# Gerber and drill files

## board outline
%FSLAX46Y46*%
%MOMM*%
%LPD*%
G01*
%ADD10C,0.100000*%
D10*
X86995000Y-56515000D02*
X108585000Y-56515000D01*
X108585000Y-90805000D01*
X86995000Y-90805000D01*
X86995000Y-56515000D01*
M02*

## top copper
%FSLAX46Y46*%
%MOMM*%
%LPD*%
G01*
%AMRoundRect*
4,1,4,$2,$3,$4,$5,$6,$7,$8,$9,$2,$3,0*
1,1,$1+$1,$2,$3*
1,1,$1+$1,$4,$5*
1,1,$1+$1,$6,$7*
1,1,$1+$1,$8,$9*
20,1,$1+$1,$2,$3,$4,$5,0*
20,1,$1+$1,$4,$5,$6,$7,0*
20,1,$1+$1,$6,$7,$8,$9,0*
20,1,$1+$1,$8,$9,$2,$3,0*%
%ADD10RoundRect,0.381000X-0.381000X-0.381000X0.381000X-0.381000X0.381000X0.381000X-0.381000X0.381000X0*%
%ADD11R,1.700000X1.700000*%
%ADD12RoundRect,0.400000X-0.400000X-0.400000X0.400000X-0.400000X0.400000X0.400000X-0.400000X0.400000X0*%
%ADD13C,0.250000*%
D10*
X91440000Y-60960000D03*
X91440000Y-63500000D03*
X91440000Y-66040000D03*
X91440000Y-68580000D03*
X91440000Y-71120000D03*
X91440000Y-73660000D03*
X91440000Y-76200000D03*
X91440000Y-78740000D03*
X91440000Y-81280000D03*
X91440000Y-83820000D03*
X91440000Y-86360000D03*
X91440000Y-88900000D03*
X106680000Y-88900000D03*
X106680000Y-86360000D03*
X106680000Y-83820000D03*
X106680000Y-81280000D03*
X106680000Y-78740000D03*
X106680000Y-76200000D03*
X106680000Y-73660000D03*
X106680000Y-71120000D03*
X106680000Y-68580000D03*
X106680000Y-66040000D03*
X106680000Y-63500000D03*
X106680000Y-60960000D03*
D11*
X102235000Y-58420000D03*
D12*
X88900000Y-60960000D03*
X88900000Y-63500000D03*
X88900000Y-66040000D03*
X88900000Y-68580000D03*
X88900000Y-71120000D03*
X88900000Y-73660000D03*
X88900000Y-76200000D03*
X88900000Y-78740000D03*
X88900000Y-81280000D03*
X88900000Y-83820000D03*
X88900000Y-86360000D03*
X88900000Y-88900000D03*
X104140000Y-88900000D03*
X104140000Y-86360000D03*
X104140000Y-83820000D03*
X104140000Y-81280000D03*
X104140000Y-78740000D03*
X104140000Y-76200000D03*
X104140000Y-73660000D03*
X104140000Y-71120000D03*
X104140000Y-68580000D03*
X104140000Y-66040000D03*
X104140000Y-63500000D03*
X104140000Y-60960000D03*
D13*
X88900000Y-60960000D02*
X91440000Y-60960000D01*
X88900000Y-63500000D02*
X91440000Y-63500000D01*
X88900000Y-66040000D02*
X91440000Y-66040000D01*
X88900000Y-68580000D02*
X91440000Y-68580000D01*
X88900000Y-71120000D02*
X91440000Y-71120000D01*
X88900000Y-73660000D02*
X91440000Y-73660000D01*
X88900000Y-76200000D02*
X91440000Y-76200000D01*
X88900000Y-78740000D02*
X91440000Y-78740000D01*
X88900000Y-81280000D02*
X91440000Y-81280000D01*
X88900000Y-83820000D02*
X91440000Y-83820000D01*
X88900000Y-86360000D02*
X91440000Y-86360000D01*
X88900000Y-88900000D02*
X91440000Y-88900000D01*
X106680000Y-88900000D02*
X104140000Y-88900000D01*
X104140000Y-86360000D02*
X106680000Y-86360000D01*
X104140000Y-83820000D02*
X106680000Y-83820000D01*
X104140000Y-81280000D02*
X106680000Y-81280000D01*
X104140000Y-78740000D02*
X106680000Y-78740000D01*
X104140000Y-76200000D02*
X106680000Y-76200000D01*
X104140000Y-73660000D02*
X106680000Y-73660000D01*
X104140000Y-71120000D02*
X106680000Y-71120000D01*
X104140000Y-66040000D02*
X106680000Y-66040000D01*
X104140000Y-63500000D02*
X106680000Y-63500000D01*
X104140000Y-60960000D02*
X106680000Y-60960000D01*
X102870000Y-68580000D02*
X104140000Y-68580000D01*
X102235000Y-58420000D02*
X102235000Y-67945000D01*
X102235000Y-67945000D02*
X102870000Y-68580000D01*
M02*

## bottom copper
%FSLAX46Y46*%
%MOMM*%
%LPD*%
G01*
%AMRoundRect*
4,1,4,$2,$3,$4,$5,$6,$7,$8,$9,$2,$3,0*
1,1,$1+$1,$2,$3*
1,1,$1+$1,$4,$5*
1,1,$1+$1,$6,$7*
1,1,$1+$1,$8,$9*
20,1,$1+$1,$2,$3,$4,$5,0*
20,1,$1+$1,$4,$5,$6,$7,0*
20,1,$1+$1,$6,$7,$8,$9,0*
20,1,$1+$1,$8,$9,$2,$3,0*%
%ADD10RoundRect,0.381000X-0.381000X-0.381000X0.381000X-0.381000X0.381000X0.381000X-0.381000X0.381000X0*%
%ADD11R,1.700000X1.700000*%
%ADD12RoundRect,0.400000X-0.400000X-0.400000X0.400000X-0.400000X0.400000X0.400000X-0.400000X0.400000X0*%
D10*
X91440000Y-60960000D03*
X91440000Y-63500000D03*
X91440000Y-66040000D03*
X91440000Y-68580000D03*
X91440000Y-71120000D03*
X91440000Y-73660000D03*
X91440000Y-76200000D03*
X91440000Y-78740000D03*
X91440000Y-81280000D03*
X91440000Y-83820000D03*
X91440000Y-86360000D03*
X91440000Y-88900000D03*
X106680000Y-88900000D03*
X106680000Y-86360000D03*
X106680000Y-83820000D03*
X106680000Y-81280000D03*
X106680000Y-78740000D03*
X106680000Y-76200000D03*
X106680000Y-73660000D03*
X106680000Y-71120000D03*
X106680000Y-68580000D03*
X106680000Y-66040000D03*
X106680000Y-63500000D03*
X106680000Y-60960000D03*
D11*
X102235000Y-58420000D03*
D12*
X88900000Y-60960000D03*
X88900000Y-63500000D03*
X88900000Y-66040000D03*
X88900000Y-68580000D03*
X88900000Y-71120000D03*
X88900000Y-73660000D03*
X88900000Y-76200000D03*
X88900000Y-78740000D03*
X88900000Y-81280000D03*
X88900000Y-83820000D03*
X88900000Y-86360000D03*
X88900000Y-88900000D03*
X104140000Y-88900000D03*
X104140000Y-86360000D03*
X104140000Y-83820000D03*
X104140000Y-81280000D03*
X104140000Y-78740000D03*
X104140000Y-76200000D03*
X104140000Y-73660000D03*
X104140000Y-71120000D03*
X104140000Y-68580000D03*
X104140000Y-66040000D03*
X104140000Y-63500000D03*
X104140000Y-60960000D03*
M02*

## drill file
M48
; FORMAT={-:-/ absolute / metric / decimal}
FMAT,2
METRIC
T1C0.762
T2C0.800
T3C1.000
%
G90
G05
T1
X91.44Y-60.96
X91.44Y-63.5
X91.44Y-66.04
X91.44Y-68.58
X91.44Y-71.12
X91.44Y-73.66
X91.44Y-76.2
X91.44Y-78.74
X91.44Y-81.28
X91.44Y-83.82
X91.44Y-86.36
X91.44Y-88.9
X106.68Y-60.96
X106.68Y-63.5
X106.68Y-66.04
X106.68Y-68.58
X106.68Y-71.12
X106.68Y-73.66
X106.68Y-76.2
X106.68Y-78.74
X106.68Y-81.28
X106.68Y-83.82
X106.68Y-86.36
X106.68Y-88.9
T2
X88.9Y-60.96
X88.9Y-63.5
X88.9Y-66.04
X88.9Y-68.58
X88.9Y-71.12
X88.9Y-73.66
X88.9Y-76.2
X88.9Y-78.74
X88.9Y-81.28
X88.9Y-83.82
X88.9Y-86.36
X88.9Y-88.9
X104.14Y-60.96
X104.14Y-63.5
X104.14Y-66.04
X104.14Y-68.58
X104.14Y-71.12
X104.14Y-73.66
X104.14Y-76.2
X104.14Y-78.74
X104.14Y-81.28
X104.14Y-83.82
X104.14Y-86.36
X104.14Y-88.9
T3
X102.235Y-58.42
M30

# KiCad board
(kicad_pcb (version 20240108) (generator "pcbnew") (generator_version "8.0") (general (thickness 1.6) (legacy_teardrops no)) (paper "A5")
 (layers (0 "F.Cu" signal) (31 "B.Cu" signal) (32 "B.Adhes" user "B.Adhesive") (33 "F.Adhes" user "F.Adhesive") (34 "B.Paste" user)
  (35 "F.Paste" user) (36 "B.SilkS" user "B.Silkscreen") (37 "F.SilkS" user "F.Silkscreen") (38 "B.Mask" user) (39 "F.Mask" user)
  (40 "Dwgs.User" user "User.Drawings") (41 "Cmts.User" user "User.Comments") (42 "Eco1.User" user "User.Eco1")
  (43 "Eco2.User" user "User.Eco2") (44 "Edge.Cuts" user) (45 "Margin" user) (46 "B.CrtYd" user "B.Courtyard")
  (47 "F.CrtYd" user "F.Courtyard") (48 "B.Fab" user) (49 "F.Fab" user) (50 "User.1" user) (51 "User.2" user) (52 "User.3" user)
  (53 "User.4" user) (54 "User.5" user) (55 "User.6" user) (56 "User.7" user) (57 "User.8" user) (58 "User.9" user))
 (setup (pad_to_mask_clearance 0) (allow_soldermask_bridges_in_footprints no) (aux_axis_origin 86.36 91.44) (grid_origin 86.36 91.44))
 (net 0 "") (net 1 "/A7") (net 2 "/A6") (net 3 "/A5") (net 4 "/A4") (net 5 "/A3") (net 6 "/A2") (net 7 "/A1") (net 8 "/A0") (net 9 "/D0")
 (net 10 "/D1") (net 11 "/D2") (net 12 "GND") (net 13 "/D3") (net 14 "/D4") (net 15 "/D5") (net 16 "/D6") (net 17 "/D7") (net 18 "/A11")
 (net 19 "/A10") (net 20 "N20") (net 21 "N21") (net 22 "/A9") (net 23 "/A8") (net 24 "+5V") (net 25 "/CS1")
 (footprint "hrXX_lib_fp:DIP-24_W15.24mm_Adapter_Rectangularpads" (layer "F.Cu") (at 91.44 60.96)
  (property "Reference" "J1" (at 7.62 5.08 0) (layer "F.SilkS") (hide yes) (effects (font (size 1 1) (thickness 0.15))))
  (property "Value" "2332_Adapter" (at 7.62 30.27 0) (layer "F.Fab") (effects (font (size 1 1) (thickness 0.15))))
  (pad "1" thru_hole roundrect (at 0 0) (size 1.524 1.524) (drill 0.762) (layers "*.Cu" "*.Mask") (remove_unused_layers no)
   (roundrect_rratio 0.25) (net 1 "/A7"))
  (pad "2" thru_hole roundrect (at 0 2.54) (size 1.524 1.524) (drill 0.762) (layers "*.Cu" "*.Mask") (remove_unused_layers no)
   (roundrect_rratio 0.25) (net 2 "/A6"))
  (pad "3" thru_hole roundrect (at 0 5.08) (size 1.524 1.524) (drill 0.762) (layers "*.Cu" "*.Mask") (remove_unused_layers no)
   (roundrect_rratio 0.25) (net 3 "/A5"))
  (pad "4" thru_hole roundrect (at 0 7.62) (size 1.524 1.524) (drill 0.762) (layers "*.Cu" "*.Mask") (remove_unused_layers no)
   (roundrect_rratio 0.25) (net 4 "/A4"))
  (pad "5" thru_hole roundrect (at 0 10.16) (size 1.524 1.524) (drill 0.762) (layers "*.Cu" "*.Mask") (remove_unused_layers no)
   (roundrect_rratio 0.25) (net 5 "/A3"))
  (pad "6" thru_hole roundrect (at 0 12.7) (size 1.524 1.524) (drill 0.762) (layers "*.Cu" "*.Mask") (remove_unused_layers no)
   (roundrect_rratio 0.25) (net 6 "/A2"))
  (pad "7" thru_hole roundrect (at 0 15.24) (size 1.524 1.524) (drill 0.762) (layers "*.Cu" "*.Mask") (remove_unused_layers no)
   (roundrect_rratio 0.25) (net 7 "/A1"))
  (pad "8" thru_hole roundrect (at 0 17.78) (size 1.524 1.524) (drill 0.762) (layers "*.Cu" "*.Mask") (remove_unused_layers no)
   (roundrect_rratio 0.25) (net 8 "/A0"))
  (pad "9" thru_hole roundrect (at 0 20.32) (size 1.524 1.524) (drill 0.762) (layers "*.Cu" "*.Mask") (remove_unused_layers no)
   (roundrect_rratio 0.25) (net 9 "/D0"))
  (pad "10" thru_hole roundrect (at 0 22.86) (size 1.524 1.524) (drill 0.762) (layers "*.Cu" "*.Mask") (remove_unused_layers no)
   (roundrect_rratio 0.25) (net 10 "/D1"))
  (pad "11" thru_hole roundrect (at 0 25.4) (size 1.524 1.524) (drill 0.762) (layers "*.Cu" "*.Mask") (remove_unused_layers no)
   (roundrect_rratio 0.25) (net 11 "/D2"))
  (pad "12" thru_hole roundrect (at 0 27.94) (size 1.524 1.524) (drill 0.762) (layers "*.Cu" "*.Mask") (remove_unused_layers no)
   (roundrect_rratio 0.25) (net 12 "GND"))
  (pad "13" thru_hole roundrect (at 15.24 27.94) (size 1.524 1.524) (drill 0.762) (layers "*.Cu" "*.Mask") (remove_unused_layers no)
   (roundrect_rratio 0.25) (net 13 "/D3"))
  (pad "14" thru_hole roundrect (at 15.24 25.4) (size 1.524 1.524) (drill 0.762) (layers "*.Cu" "*.Mask") (remove_unused_layers no)
   (roundrect_rratio 0.25) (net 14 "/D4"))
  (pad "15" thru_hole roundrect (at 15.24 22.86) (size 1.524 1.524) (drill 0.762) (layers "*.Cu" "*.Mask") (remove_unused_layers no)
   (roundrect_rratio 0.25) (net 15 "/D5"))
  (pad "16" thru_hole roundrect (at 15.24 20.32) (size 1.524 1.524) (drill 0.762) (layers "*.Cu" "*.Mask") (remove_unused_layers no)
   (roundrect_rratio 0.25) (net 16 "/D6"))
  (pad "17" thru_hole roundrect (at 15.24 17.78) (size 1.524 1.524) (drill 0.762) (layers "*.Cu" "*.Mask") (remove_unused_layers no)
   (roundrect_rratio 0.25) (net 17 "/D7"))
  (pad "18" thru_hole roundrect (at 15.24 15.24) (size 1.524 1.524) (drill 0.762) (layers "*.Cu" "*.Mask") (remove_unused_layers no)
   (roundrect_rratio 0.25) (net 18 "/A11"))
  (pad "19" thru_hole roundrect (at 15.24 12.7) (size 1.524 1.524) (drill 0.762) (layers "*.Cu" "*.Mask") (remove_unused_layers no)
   (roundrect_rratio 0.25) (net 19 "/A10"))
  (pad "20" thru_hole roundrect (at 15.24 10.16) (size 1.524 1.524) (drill 0.762) (layers "*.Cu" "*.Mask") (remove_unused_layers no)
   (roundrect_rratio 0.25) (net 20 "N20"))
  (pad "21" thru_hole roundrect (at 15.24 7.62) (size 1.524 1.524) (drill 0.762) (layers "*.Cu" "*.Mask") (remove_unused_layers no)
   (roundrect_rratio 0.25) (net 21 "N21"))
  (pad "22" thru_hole roundrect (at 15.24 5.08) (size 1.524 1.524) (drill 0.762) (layers "*.Cu" "*.Mask") (remove_unused_layers no)
   (roundrect_rratio 0.25) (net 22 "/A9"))
  (pad "23" thru_hole roundrect (at 15.24 2.54) (size 1.524 1.524) (drill 0.762) (layers "*.Cu" "*.Mask") (remove_unused_layers no)
   (roundrect_rratio 0.25) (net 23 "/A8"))
  (pad "24" thru_hole roundrect (at 15.24 0) (size 1.524 1.524) (drill 0.762) (layers "*.Cu" "*.Mask") (remove_unused_layers no)
   (roundrect_rratio 0.25) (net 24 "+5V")))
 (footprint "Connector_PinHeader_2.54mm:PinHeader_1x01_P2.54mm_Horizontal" (layer "F.Cu") (at 102.235 58.42 180)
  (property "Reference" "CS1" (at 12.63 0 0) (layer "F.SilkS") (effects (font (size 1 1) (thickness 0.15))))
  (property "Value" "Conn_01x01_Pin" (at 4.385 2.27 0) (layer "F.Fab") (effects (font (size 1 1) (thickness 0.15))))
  (pad "1" thru_hole rect (at 0 0 180) (size 1.7 1.7) (drill 1) (layers "*.Cu" "*.Mask") (remove_unused_layers no) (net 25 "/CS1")))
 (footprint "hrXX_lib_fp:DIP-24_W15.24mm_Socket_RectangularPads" (layer "F.Cu") (at 88.9 60.96)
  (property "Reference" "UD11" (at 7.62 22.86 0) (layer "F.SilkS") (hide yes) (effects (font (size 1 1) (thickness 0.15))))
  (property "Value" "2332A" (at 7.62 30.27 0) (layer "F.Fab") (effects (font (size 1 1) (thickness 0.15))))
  (pad "1" thru_hole roundrect (at 0 0) (size 1.6 1.6) (drill 0.8) (layers "*.Cu" "*.Mask") (remove_unused_layers no)
   (roundrect_rratio 0.25) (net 1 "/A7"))
  (pad "2" thru_hole roundrect (at 0 2.54) (size 1.6 1.6) (drill 0.8) (layers "*.Cu" "*.Mask") (remove_unused_layers no)
   (roundrect_rratio 0.25) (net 2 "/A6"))
  (pad "3" thru_hole roundrect (at 0 5.08) (size 1.6 1.6) (drill 0.8) (layers "*.Cu" "*.Mask") (remove_unused_layers no)
   (roundrect_rratio 0.25) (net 3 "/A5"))
  (pad "4" thru_hole roundrect (at 0 7.62) (size 1.6 1.6) (drill 0.8) (layers "*.Cu" "*.Mask") (remove_unused_layers no)
   (roundrect_rratio 0.25) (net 4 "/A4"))
  (pad "5" thru_hole roundrect (at 0 10.16) (size 1.6 1.6) (drill 0.8) (layers "*.Cu" "*.Mask") (remove_unused_layers no)
   (roundrect_rratio 0.25) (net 5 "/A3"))
  (pad "6" thru_hole roundrect (at 0 12.7) (size 1.6 1.6) (drill 0.8) (layers "*.Cu" "*.Mask") (remove_unused_layers no)
   (roundrect_rratio 0.25) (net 6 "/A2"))
  (pad "7" thru_hole roundrect (at 0 15.24) (size 1.6 1.6) (drill 0.8) (layers "*.Cu" "*.Mask") (remove_unused_layers no)
   (roundrect_rratio 0.25) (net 7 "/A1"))
  (pad "8" thru_hole roundrect (at 0 17.78) (size 1.6 1.6) (drill 0.8) (layers "*.Cu" "*.Mask") (remove_unused_layers no)
   (roundrect_rratio 0.25) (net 8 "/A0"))
  (pad "9" thru_hole roundrect (at 0 20.32) (size 1.6 1.6) (drill 0.8) (layers "*.Cu" "*.Mask") (remove_unused_layers no)
   (roundrect_rratio 0.25) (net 9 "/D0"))
  (pad "10" thru_hole roundrect (at 0 22.86) (size 1.6 1.6) (drill 0.8) (layers "*.Cu" "*.Mask") (remove_unused_layers no)
   (roundrect_rratio 0.25) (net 10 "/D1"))
  (pad "11" thru_hole roundrect (at 0 25.4) (size 1.6 1.6) (drill 0.8) (layers "*.Cu" "*.Mask") (remove_unused_layers no)
   (roundrect_rratio 0.25) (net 11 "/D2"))
  (pad "12" thru_hole roundrect (at 0 27.94) (size 1.6 1.6) (drill 0.8) (layers "*.Cu" "*.Mask") (remove_unused_layers no)
   (roundrect_rratio 0.25) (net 12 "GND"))
  (pad "13" thru_hole roundrect (at 15.24 27.94) (size 1.6 1.6) (drill 0.8) (layers "*.Cu" "*.Mask") (remove_unused_layers no)
   (roundrect_rratio 0.25) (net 13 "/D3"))
  (pad "14" thru_hole roundrect (at 15.24 25.4) (size 1.6 1.6) (drill 0.8) (layers "*.Cu" "*.Mask") (remove_unused_layers no)
   (roundrect_rratio 0.25) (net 14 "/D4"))
  (pad "15" thru_hole roundrect (at 15.24 22.86) (size 1.6 1.6) (drill 0.8) (layers "*.Cu" "*.Mask") (remove_unused_layers no)
   (roundrect_rratio 0.25) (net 15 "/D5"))
  (pad "16" thru_hole roundrect (at 15.24 20.32) (size 1.6 1.6) (drill 0.8) (layers "*.Cu" "*.Mask") (remove_unused_layers no)
   (roundrect_rratio 0.25) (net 16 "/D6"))
  (pad "17" thru_hole roundrect (at 15.24 17.78) (size 1.6 1.6) (drill 0.8) (layers "*.Cu" "*.Mask") (remove_unused_layers no)
   (roundrect_rratio 0.25) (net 17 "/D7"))
  (pad "18" thru_hole roundrect (at 15.24 15.24) (size 1.6 1.6) (drill 0.8) (layers "*.Cu" "*.Mask") (remove_unused_layers no)
   (roundrect_rratio 0.25) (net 18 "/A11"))
  (pad "19" thru_hole roundrect (at 15.24 12.7) (size 1.6 1.6) (drill 0.8) (layers "*.Cu" "*.Mask") (remove_unused_layers no)
   (roundrect_rratio 0.25) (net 19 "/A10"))
  (pad "20" thru_hole roundrect (at 15.24 10.16) (size 1.6 1.6) (drill 0.8) (layers "*.Cu" "*.Mask") (remove_unused_layers no)
   (roundrect_rratio 0.25) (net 20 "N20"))
  (pad "21" thru_hole roundrect (at 15.24 7.62) (size 1.6 1.6) (drill 0.8) (layers "*.Cu" "*.Mask") (remove_unused_layers no)
   (roundrect_rratio 0.25) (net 25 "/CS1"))
  (pad "22" thru_hole roundrect (at 15.24 5.08) (size 1.6 1.6) (drill 0.8) (layers "*.Cu" "*.Mask") (remove_unused_layers no)
   (roundrect_rratio 0.25) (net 22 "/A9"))
  (pad "23" thru_hole roundrect (at 15.24 2.54) (size 1.6 1.6) (drill 0.8) (layers "*.Cu" "*.Mask") (remove_unused_layers no)
   (roundrect_rratio 0.25) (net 23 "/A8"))
  (pad "24" thru_hole roundrect (at 15.24 0) (size 1.6 1.6) (drill 0.8) (layers "*.Cu" "*.Mask") (remove_unused_layers no)
   (roundrect_rratio 0.25) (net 24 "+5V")))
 (gr_rect (start 86.995 56.515) (end 108.585 90.805) (stroke (width 0.1) (type solid)) (fill none) (layer "Edge.Cuts"))
 (segment (start 88.9 60.96) (end 91.44 60.96) (width 0.25) (layer "F.Cu") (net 1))
 (segment (start 88.9 63.5) (end 91.44 63.5) (width 0.25) (layer "F.Cu") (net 2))
 (segment (start 88.9 66.04) (end 91.44 66.04) (width 0.25) (layer "F.Cu") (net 3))
 (segment (start 88.9 68.58) (end 91.44 68.58) (width 0.25) (layer "F.Cu") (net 4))
 (segment (start 88.9 71.12) (end 91.44 71.12) (width 0.25) (layer "F.Cu") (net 5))
 (segment (start 88.9 73.66) (end 91.44 73.66) (width 0.25) (layer "F.Cu") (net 6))
 (segment (start 88.9 76.2) (end 91.44 76.2) (width 0.25) (layer "F.Cu") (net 7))
 (segment (start 88.9 78.74) (end 91.44 78.74) (width 0.25) (layer "F.Cu") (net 8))
 (segment (start 88.9 81.28) (end 91.44 81.28) (width 0.25) (layer "F.Cu") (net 9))
 (segment (start 88.9 83.82) (end 91.44 83.82) (width 0.25) (layer "F.Cu") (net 10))
 (segment (start 88.9 86.36) (end 91.44 86.36) (width 0.25) (layer "F.Cu") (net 11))
 (segment (start 88.9 88.9) (end 91.44 88.9) (width 0.25) (layer "F.Cu") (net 12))
 (segment (start 106.68 88.9) (end 104.14 88.9) (width 0.25) (layer "F.Cu") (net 13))
 (segment (start 104.14 86.36) (end 106.68 86.36) (width 0.25) (layer "F.Cu") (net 14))
 (segment (start 104.14 83.82) (end 106.68 83.82) (width 0.25) (layer "F.Cu") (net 15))
 (segment (start 104.14 81.28) (end 106.68 81.28) (width 0.25) (layer "F.Cu") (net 16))
 (segment (start 104.14 78.74) (end 106.68 78.74) (width 0.25) (layer "F.Cu") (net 17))
 (segment (start 104.14 76.2) (end 106.68 76.2) (width 0.25) (layer "F.Cu") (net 18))
 (segment (start 104.14 73.66) (end 106.68 73.66) (width 0.25) (layer "F.Cu") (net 19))
 (segment (start 104.14 71.12) (end 106.68 71.12) (width 0.25) (layer "F.Cu") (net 20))
 (segment (start 104.14 66.04) (end 106.68 66.04) (width 0.25) (layer "F.Cu") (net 22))
 (segment (start 104.14 63.5) (end 106.68 63.5) (width 0.25) (layer "F.Cu") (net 23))
 (segment (start 104.14 60.96) (end 106.68 60.96) (width 0.25) (layer "F.Cu") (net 24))
 (segment (start 102.87 68.58) (end 104.14 68.58) (width 0.25) (layer "F.Cu") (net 25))
 (segment (start 102.235 58.42) (end 102.235 67.945) (width 0.25) (layer "F.Cu") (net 25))
 (segment (start 102.235 67.945) (end 102.87 68.58) (width 0.25) (layer "F.Cu") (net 25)))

